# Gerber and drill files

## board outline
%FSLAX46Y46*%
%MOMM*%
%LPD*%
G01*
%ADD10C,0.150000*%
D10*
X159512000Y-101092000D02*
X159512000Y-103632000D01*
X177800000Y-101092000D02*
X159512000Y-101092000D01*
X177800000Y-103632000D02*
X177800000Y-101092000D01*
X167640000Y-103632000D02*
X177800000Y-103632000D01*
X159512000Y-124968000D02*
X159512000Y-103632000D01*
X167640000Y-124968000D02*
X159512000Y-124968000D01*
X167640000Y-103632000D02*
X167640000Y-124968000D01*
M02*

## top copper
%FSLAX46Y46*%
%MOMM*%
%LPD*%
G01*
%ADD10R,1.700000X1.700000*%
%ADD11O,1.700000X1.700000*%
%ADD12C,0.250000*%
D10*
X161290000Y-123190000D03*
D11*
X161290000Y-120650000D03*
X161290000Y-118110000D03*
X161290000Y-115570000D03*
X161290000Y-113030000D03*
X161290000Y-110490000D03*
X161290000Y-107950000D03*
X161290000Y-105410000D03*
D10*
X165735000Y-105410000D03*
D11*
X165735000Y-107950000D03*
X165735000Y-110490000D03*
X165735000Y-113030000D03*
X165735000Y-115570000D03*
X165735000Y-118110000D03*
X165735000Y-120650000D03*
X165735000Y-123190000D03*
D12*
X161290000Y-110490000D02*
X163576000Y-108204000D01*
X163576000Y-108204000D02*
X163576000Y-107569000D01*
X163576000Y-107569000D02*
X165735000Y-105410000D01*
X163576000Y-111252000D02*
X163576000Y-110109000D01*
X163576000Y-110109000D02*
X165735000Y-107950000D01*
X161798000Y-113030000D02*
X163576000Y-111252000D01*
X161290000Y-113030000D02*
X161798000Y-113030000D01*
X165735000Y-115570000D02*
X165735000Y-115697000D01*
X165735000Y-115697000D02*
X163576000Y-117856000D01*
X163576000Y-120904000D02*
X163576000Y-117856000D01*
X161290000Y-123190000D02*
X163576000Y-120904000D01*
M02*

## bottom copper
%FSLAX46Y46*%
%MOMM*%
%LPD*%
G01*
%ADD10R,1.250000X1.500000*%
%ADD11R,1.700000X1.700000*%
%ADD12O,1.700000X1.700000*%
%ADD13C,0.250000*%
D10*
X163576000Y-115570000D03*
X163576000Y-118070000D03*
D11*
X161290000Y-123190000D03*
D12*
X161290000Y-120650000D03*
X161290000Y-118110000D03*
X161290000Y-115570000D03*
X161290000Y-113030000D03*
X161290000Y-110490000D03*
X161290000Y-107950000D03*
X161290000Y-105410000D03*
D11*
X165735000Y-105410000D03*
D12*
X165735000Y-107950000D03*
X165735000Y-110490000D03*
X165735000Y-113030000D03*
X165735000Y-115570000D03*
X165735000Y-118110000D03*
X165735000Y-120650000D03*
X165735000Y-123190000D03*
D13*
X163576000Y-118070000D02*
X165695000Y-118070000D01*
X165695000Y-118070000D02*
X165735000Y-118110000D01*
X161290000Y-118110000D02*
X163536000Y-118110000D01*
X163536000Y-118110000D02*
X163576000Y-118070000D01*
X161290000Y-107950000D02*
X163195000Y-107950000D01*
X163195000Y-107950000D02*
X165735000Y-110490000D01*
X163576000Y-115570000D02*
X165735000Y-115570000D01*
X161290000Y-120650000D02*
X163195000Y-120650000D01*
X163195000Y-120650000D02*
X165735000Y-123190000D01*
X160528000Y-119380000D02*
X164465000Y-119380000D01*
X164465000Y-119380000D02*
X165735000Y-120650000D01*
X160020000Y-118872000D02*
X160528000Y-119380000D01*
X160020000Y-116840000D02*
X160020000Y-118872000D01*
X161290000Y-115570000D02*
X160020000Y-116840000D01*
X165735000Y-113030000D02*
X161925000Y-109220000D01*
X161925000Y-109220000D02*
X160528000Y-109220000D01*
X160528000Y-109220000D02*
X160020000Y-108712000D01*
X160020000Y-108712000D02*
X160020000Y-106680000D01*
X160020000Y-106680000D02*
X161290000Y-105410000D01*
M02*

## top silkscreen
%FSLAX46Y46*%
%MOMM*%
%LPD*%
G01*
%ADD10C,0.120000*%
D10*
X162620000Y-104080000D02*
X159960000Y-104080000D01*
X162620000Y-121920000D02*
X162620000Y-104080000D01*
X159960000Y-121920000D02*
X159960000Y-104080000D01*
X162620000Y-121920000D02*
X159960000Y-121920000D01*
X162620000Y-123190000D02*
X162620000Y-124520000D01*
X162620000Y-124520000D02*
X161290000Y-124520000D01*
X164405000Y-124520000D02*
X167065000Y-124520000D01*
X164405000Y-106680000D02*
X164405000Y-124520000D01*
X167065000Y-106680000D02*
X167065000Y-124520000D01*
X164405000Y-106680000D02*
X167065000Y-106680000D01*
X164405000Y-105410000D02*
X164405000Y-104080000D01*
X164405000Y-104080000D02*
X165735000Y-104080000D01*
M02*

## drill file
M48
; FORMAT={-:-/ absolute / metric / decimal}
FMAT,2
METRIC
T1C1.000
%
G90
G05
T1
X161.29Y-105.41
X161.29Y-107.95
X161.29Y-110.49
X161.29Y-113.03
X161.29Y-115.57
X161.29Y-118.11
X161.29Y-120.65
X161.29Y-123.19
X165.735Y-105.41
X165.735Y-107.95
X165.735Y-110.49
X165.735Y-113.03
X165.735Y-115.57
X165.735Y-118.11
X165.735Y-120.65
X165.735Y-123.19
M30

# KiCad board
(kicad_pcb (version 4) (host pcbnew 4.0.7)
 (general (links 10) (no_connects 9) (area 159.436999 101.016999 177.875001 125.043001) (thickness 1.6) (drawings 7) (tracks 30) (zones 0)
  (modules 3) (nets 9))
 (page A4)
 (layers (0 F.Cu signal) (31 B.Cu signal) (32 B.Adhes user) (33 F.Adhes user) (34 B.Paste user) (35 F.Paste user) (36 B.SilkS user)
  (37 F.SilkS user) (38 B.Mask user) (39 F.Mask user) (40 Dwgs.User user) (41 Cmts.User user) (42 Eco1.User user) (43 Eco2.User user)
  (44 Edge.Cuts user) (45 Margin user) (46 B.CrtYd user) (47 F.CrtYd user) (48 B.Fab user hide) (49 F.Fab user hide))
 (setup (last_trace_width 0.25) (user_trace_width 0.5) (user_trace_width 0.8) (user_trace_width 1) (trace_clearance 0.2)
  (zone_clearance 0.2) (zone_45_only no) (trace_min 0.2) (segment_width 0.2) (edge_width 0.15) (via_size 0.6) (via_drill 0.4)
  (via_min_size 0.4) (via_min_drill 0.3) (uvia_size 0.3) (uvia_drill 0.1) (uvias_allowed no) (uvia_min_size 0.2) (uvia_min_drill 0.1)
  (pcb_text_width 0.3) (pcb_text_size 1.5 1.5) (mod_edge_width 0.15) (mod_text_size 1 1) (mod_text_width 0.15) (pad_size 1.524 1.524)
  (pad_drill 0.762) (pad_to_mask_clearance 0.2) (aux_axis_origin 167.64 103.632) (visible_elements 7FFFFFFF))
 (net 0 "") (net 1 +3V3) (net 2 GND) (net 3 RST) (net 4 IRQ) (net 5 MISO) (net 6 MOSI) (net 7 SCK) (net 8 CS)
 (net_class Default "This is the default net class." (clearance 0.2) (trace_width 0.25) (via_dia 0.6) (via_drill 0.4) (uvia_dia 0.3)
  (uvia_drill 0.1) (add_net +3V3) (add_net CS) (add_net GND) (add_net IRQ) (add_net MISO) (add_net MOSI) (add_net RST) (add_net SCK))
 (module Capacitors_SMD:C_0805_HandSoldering (layer B.Cu) (at 163.576 116.82 270)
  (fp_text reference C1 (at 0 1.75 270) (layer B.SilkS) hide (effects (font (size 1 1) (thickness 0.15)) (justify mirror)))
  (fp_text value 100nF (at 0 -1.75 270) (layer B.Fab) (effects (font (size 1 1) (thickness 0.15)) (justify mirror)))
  (pad 1 smd rect (at -1.25 0 270) (size 1.5 1.25) (layers B.Cu B.Paste B.Mask) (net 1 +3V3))
  (pad 2 smd rect (at 1.25 0 270) (size 1.5 1.25) (layers B.Cu B.Paste B.Mask) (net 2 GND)))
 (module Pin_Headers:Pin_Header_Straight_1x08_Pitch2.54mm (layer F.Cu) (at 161.29 123.19 180)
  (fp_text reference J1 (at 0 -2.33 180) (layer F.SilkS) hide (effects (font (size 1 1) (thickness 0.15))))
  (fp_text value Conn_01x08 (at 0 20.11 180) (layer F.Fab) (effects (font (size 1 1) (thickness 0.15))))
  (fp_line (start -1.33 19.11) (end 1.33 19.11) (layer F.SilkS) (width 0.12))
  (fp_line (start -1.33 1.27) (end -1.33 19.11) (layer F.SilkS) (width 0.12))
  (fp_line (start 1.33 1.27) (end 1.33 19.11) (layer F.SilkS) (width 0.12))
  (fp_line (start -1.33 1.27) (end 1.33 1.27) (layer F.SilkS) (width 0.12))
  (fp_line (start -1.33 0) (end -1.33 -1.33) (layer F.SilkS) (width 0.12))
  (fp_line (start -1.33 -1.33) (end 0 -1.33) (layer F.SilkS) (width 0.12))
  (pad 1 thru_hole rect (at 0 0 180) (size 1.7 1.7) (drill 1) (layers *.Cu *.Mask) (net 1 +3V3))
  (pad 2 thru_hole oval (at 0 2.54 180) (size 1.7 1.7) (drill 1) (layers *.Cu *.Mask) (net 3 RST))
  (pad 3 thru_hole oval (at 0 5.08 180) (size 1.7 1.7) (drill 1) (layers *.Cu *.Mask) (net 2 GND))
  (pad 4 thru_hole oval (at 0 7.62 180) (size 1.7 1.7) (drill 1) (layers *.Cu *.Mask) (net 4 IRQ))
  (pad 5 thru_hole oval (at 0 10.16 180) (size 1.7 1.7) (drill 1) (layers *.Cu *.Mask) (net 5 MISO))
  (pad 6 thru_hole oval (at 0 12.7 180) (size 1.7 1.7) (drill 1) (layers *.Cu *.Mask) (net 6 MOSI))
  (pad 7 thru_hole oval (at 0 15.24 180) (size 1.7 1.7) (drill 1) (layers *.Cu *.Mask) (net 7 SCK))
  (pad 8 thru_hole oval (at 0 17.78 180) (size 1.7 1.7) (drill 1) (layers *.Cu *.Mask) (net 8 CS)))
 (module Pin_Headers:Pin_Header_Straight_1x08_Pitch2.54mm (layer F.Cu) (at 165.735 105.41)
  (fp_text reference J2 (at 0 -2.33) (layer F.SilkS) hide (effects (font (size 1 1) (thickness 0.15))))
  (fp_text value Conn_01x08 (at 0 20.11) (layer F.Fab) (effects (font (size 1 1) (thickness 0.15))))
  (fp_line (start -1.33 19.11) (end 1.33 19.11) (layer F.SilkS) (width 0.12))
  (fp_line (start -1.33 1.27) (end -1.33 19.11) (layer F.SilkS) (width 0.12))
  (fp_line (start 1.33 1.27) (end 1.33 19.11) (layer F.SilkS) (width 0.12))
  (fp_line (start -1.33 1.27) (end 1.33 1.27) (layer F.SilkS) (width 0.12))
  (fp_line (start -1.33 0) (end -1.33 -1.33) (layer F.SilkS) (width 0.12))
  (fp_line (start -1.33 -1.33) (end 0 -1.33) (layer F.SilkS) (width 0.12))
  (pad 1 thru_hole rect (at 0 0) (size 1.7 1.7) (drill 1) (layers *.Cu *.Mask) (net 6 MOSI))
  (pad 2 thru_hole oval (at 0 2.54) (size 1.7 1.7) (drill 1) (layers *.Cu *.Mask) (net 5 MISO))
  (pad 3 thru_hole oval (at 0 5.08) (size 1.7 1.7) (drill 1) (layers *.Cu *.Mask) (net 7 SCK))
  (pad 4 thru_hole oval (at 0 7.62) (size 1.7 1.7) (drill 1) (layers *.Cu *.Mask) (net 8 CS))
  (pad 5 thru_hole oval (at 0 10.16) (size 1.7 1.7) (drill 1) (layers *.Cu *.Mask) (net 1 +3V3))
  (pad 6 thru_hole oval (at 0 12.7) (size 1.7 1.7) (drill 1) (layers *.Cu *.Mask) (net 2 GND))
  (pad 7 thru_hole oval (at 0 15.24) (size 1.7 1.7) (drill 1) (layers *.Cu *.Mask) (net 4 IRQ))
  (pad 8 thru_hole oval (at 0 17.78) (size 1.7 1.7) (drill 1) (layers *.Cu *.Mask) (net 3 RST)))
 (gr_line (start 159.512 101.092) (end 159.512 103.632) (layer Edge.Cuts) (width 0.15))
 (gr_line (start 177.8 101.092) (end 159.512 101.092) (layer Edge.Cuts) (width 0.15))
 (gr_line (start 177.8 103.632) (end 177.8 101.092) (layer Edge.Cuts) (width 0.15))
 (gr_line (start 167.64 103.632) (end 177.8 103.632) (layer Edge.Cuts) (width 0.15))
 (gr_line (start 159.512 124.968) (end 159.512 103.632) (layer Edge.Cuts) (width 0.15))
 (gr_line (start 167.64 124.968) (end 159.512 124.968) (layer Edge.Cuts) (width 0.15))
 (gr_line (start 167.64 103.632) (end 167.64 124.968) (layer Edge.Cuts) (width 0.15))
 (segment (start 163.576 118.07) (end 165.695 118.07) (width 0.25) (layer B.Cu) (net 2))
 (segment (start 165.695 118.07) (end 165.735 118.11) (width 0.25) (layer B.Cu) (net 2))
 (segment (start 161.29 118.11) (end 163.536 118.11) (width 0.25) (layer B.Cu) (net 2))
 (segment (start 163.536 118.11) (end 163.576 118.07) (width 0.25) (layer B.Cu) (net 2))
 (segment (start 161.29 110.49) (end 163.576 108.204) (width 0.25) (layer F.Cu) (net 6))
 (segment (start 163.576 108.204) (end 163.576 107.569) (width 0.25) (layer F.Cu) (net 6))
 (segment (start 163.576 107.569) (end 165.735 105.41) (width 0.25) (layer F.Cu) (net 6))
 (segment (start 163.576 111.252) (end 163.576 110.109) (width 0.25) (layer F.Cu) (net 5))
 (segment (start 163.576 110.109) (end 165.735 107.95) (width 0.25) (layer F.Cu) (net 5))
 (segment (start 161.798 113.03) (end 163.576 111.252) (width 0.25) (layer F.Cu) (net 5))
 (segment (start 161.29 113.03) (end 161.798 113.03) (width 0.25) (layer F.Cu) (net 5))
 (segment (start 161.29 107.95) (end 163.195 107.95) (width 0.25) (layer B.Cu) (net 7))
 (segment (start 163.195 107.95) (end 165.735 110.49) (width 0.25) (layer B.Cu) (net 7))
 (segment (start 165.735 115.57) (end 165.735 115.697) (width 0.25) (layer F.Cu) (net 1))
 (segment (start 165.735 115.697) (end 163.576 117.856) (width 0.25) (layer F.Cu) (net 1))
 (segment (start 163.576 120.904) (end 163.576 117.856) (width 0.25) (layer F.Cu) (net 1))
 (segment (start 161.29 123.19) (end 163.576 120.904) (width 0.25) (layer F.Cu) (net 1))
 (segment (start 163.576 115.57) (end 165.735 115.57) (width 0.25) (layer B.Cu) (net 1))
 (segment (start 161.29 120.65) (end 163.195 120.65) (width 0.25) (layer B.Cu) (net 3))
 (segment (start 163.195 120.65) (end 165.735 123.19) (width 0.25) (layer B.Cu) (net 3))
 (segment (start 160.528 119.38) (end 164.465 119.38) (width 0.25) (layer B.Cu) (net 4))
 (segment (start 164.465 119.38) (end 165.735 120.65) (width 0.25) (layer B.Cu) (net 4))
 (segment (start 160.02 118.872) (end 160.528 119.38) (width 0.25) (layer B.Cu) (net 4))
 (segment (start 160.02 116.84) (end 160.02 118.872) (width 0.25) (layer B.Cu) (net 4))
 (segment (start 161.29 115.57) (end 160.02 116.84) (width 0.25) (layer B.Cu) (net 4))
 (segment (start 165.735 113.03) (end 161.925 109.22) (width 0.25) (layer B.Cu) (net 8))
 (segment (start 161.925 109.22) (end 160.528 109.22) (width 0.25) (layer B.Cu) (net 8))
 (segment (start 160.528 109.22) (end 160.02 108.712) (width 0.25) (layer B.Cu) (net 8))
 (segment (start 160.02 108.712) (end 160.02 106.68) (width 0.25) (layer B.Cu) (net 8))
 (segment (start 160.02 106.68) (end 161.29 105.41) (width 0.25) (layer B.Cu) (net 8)))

